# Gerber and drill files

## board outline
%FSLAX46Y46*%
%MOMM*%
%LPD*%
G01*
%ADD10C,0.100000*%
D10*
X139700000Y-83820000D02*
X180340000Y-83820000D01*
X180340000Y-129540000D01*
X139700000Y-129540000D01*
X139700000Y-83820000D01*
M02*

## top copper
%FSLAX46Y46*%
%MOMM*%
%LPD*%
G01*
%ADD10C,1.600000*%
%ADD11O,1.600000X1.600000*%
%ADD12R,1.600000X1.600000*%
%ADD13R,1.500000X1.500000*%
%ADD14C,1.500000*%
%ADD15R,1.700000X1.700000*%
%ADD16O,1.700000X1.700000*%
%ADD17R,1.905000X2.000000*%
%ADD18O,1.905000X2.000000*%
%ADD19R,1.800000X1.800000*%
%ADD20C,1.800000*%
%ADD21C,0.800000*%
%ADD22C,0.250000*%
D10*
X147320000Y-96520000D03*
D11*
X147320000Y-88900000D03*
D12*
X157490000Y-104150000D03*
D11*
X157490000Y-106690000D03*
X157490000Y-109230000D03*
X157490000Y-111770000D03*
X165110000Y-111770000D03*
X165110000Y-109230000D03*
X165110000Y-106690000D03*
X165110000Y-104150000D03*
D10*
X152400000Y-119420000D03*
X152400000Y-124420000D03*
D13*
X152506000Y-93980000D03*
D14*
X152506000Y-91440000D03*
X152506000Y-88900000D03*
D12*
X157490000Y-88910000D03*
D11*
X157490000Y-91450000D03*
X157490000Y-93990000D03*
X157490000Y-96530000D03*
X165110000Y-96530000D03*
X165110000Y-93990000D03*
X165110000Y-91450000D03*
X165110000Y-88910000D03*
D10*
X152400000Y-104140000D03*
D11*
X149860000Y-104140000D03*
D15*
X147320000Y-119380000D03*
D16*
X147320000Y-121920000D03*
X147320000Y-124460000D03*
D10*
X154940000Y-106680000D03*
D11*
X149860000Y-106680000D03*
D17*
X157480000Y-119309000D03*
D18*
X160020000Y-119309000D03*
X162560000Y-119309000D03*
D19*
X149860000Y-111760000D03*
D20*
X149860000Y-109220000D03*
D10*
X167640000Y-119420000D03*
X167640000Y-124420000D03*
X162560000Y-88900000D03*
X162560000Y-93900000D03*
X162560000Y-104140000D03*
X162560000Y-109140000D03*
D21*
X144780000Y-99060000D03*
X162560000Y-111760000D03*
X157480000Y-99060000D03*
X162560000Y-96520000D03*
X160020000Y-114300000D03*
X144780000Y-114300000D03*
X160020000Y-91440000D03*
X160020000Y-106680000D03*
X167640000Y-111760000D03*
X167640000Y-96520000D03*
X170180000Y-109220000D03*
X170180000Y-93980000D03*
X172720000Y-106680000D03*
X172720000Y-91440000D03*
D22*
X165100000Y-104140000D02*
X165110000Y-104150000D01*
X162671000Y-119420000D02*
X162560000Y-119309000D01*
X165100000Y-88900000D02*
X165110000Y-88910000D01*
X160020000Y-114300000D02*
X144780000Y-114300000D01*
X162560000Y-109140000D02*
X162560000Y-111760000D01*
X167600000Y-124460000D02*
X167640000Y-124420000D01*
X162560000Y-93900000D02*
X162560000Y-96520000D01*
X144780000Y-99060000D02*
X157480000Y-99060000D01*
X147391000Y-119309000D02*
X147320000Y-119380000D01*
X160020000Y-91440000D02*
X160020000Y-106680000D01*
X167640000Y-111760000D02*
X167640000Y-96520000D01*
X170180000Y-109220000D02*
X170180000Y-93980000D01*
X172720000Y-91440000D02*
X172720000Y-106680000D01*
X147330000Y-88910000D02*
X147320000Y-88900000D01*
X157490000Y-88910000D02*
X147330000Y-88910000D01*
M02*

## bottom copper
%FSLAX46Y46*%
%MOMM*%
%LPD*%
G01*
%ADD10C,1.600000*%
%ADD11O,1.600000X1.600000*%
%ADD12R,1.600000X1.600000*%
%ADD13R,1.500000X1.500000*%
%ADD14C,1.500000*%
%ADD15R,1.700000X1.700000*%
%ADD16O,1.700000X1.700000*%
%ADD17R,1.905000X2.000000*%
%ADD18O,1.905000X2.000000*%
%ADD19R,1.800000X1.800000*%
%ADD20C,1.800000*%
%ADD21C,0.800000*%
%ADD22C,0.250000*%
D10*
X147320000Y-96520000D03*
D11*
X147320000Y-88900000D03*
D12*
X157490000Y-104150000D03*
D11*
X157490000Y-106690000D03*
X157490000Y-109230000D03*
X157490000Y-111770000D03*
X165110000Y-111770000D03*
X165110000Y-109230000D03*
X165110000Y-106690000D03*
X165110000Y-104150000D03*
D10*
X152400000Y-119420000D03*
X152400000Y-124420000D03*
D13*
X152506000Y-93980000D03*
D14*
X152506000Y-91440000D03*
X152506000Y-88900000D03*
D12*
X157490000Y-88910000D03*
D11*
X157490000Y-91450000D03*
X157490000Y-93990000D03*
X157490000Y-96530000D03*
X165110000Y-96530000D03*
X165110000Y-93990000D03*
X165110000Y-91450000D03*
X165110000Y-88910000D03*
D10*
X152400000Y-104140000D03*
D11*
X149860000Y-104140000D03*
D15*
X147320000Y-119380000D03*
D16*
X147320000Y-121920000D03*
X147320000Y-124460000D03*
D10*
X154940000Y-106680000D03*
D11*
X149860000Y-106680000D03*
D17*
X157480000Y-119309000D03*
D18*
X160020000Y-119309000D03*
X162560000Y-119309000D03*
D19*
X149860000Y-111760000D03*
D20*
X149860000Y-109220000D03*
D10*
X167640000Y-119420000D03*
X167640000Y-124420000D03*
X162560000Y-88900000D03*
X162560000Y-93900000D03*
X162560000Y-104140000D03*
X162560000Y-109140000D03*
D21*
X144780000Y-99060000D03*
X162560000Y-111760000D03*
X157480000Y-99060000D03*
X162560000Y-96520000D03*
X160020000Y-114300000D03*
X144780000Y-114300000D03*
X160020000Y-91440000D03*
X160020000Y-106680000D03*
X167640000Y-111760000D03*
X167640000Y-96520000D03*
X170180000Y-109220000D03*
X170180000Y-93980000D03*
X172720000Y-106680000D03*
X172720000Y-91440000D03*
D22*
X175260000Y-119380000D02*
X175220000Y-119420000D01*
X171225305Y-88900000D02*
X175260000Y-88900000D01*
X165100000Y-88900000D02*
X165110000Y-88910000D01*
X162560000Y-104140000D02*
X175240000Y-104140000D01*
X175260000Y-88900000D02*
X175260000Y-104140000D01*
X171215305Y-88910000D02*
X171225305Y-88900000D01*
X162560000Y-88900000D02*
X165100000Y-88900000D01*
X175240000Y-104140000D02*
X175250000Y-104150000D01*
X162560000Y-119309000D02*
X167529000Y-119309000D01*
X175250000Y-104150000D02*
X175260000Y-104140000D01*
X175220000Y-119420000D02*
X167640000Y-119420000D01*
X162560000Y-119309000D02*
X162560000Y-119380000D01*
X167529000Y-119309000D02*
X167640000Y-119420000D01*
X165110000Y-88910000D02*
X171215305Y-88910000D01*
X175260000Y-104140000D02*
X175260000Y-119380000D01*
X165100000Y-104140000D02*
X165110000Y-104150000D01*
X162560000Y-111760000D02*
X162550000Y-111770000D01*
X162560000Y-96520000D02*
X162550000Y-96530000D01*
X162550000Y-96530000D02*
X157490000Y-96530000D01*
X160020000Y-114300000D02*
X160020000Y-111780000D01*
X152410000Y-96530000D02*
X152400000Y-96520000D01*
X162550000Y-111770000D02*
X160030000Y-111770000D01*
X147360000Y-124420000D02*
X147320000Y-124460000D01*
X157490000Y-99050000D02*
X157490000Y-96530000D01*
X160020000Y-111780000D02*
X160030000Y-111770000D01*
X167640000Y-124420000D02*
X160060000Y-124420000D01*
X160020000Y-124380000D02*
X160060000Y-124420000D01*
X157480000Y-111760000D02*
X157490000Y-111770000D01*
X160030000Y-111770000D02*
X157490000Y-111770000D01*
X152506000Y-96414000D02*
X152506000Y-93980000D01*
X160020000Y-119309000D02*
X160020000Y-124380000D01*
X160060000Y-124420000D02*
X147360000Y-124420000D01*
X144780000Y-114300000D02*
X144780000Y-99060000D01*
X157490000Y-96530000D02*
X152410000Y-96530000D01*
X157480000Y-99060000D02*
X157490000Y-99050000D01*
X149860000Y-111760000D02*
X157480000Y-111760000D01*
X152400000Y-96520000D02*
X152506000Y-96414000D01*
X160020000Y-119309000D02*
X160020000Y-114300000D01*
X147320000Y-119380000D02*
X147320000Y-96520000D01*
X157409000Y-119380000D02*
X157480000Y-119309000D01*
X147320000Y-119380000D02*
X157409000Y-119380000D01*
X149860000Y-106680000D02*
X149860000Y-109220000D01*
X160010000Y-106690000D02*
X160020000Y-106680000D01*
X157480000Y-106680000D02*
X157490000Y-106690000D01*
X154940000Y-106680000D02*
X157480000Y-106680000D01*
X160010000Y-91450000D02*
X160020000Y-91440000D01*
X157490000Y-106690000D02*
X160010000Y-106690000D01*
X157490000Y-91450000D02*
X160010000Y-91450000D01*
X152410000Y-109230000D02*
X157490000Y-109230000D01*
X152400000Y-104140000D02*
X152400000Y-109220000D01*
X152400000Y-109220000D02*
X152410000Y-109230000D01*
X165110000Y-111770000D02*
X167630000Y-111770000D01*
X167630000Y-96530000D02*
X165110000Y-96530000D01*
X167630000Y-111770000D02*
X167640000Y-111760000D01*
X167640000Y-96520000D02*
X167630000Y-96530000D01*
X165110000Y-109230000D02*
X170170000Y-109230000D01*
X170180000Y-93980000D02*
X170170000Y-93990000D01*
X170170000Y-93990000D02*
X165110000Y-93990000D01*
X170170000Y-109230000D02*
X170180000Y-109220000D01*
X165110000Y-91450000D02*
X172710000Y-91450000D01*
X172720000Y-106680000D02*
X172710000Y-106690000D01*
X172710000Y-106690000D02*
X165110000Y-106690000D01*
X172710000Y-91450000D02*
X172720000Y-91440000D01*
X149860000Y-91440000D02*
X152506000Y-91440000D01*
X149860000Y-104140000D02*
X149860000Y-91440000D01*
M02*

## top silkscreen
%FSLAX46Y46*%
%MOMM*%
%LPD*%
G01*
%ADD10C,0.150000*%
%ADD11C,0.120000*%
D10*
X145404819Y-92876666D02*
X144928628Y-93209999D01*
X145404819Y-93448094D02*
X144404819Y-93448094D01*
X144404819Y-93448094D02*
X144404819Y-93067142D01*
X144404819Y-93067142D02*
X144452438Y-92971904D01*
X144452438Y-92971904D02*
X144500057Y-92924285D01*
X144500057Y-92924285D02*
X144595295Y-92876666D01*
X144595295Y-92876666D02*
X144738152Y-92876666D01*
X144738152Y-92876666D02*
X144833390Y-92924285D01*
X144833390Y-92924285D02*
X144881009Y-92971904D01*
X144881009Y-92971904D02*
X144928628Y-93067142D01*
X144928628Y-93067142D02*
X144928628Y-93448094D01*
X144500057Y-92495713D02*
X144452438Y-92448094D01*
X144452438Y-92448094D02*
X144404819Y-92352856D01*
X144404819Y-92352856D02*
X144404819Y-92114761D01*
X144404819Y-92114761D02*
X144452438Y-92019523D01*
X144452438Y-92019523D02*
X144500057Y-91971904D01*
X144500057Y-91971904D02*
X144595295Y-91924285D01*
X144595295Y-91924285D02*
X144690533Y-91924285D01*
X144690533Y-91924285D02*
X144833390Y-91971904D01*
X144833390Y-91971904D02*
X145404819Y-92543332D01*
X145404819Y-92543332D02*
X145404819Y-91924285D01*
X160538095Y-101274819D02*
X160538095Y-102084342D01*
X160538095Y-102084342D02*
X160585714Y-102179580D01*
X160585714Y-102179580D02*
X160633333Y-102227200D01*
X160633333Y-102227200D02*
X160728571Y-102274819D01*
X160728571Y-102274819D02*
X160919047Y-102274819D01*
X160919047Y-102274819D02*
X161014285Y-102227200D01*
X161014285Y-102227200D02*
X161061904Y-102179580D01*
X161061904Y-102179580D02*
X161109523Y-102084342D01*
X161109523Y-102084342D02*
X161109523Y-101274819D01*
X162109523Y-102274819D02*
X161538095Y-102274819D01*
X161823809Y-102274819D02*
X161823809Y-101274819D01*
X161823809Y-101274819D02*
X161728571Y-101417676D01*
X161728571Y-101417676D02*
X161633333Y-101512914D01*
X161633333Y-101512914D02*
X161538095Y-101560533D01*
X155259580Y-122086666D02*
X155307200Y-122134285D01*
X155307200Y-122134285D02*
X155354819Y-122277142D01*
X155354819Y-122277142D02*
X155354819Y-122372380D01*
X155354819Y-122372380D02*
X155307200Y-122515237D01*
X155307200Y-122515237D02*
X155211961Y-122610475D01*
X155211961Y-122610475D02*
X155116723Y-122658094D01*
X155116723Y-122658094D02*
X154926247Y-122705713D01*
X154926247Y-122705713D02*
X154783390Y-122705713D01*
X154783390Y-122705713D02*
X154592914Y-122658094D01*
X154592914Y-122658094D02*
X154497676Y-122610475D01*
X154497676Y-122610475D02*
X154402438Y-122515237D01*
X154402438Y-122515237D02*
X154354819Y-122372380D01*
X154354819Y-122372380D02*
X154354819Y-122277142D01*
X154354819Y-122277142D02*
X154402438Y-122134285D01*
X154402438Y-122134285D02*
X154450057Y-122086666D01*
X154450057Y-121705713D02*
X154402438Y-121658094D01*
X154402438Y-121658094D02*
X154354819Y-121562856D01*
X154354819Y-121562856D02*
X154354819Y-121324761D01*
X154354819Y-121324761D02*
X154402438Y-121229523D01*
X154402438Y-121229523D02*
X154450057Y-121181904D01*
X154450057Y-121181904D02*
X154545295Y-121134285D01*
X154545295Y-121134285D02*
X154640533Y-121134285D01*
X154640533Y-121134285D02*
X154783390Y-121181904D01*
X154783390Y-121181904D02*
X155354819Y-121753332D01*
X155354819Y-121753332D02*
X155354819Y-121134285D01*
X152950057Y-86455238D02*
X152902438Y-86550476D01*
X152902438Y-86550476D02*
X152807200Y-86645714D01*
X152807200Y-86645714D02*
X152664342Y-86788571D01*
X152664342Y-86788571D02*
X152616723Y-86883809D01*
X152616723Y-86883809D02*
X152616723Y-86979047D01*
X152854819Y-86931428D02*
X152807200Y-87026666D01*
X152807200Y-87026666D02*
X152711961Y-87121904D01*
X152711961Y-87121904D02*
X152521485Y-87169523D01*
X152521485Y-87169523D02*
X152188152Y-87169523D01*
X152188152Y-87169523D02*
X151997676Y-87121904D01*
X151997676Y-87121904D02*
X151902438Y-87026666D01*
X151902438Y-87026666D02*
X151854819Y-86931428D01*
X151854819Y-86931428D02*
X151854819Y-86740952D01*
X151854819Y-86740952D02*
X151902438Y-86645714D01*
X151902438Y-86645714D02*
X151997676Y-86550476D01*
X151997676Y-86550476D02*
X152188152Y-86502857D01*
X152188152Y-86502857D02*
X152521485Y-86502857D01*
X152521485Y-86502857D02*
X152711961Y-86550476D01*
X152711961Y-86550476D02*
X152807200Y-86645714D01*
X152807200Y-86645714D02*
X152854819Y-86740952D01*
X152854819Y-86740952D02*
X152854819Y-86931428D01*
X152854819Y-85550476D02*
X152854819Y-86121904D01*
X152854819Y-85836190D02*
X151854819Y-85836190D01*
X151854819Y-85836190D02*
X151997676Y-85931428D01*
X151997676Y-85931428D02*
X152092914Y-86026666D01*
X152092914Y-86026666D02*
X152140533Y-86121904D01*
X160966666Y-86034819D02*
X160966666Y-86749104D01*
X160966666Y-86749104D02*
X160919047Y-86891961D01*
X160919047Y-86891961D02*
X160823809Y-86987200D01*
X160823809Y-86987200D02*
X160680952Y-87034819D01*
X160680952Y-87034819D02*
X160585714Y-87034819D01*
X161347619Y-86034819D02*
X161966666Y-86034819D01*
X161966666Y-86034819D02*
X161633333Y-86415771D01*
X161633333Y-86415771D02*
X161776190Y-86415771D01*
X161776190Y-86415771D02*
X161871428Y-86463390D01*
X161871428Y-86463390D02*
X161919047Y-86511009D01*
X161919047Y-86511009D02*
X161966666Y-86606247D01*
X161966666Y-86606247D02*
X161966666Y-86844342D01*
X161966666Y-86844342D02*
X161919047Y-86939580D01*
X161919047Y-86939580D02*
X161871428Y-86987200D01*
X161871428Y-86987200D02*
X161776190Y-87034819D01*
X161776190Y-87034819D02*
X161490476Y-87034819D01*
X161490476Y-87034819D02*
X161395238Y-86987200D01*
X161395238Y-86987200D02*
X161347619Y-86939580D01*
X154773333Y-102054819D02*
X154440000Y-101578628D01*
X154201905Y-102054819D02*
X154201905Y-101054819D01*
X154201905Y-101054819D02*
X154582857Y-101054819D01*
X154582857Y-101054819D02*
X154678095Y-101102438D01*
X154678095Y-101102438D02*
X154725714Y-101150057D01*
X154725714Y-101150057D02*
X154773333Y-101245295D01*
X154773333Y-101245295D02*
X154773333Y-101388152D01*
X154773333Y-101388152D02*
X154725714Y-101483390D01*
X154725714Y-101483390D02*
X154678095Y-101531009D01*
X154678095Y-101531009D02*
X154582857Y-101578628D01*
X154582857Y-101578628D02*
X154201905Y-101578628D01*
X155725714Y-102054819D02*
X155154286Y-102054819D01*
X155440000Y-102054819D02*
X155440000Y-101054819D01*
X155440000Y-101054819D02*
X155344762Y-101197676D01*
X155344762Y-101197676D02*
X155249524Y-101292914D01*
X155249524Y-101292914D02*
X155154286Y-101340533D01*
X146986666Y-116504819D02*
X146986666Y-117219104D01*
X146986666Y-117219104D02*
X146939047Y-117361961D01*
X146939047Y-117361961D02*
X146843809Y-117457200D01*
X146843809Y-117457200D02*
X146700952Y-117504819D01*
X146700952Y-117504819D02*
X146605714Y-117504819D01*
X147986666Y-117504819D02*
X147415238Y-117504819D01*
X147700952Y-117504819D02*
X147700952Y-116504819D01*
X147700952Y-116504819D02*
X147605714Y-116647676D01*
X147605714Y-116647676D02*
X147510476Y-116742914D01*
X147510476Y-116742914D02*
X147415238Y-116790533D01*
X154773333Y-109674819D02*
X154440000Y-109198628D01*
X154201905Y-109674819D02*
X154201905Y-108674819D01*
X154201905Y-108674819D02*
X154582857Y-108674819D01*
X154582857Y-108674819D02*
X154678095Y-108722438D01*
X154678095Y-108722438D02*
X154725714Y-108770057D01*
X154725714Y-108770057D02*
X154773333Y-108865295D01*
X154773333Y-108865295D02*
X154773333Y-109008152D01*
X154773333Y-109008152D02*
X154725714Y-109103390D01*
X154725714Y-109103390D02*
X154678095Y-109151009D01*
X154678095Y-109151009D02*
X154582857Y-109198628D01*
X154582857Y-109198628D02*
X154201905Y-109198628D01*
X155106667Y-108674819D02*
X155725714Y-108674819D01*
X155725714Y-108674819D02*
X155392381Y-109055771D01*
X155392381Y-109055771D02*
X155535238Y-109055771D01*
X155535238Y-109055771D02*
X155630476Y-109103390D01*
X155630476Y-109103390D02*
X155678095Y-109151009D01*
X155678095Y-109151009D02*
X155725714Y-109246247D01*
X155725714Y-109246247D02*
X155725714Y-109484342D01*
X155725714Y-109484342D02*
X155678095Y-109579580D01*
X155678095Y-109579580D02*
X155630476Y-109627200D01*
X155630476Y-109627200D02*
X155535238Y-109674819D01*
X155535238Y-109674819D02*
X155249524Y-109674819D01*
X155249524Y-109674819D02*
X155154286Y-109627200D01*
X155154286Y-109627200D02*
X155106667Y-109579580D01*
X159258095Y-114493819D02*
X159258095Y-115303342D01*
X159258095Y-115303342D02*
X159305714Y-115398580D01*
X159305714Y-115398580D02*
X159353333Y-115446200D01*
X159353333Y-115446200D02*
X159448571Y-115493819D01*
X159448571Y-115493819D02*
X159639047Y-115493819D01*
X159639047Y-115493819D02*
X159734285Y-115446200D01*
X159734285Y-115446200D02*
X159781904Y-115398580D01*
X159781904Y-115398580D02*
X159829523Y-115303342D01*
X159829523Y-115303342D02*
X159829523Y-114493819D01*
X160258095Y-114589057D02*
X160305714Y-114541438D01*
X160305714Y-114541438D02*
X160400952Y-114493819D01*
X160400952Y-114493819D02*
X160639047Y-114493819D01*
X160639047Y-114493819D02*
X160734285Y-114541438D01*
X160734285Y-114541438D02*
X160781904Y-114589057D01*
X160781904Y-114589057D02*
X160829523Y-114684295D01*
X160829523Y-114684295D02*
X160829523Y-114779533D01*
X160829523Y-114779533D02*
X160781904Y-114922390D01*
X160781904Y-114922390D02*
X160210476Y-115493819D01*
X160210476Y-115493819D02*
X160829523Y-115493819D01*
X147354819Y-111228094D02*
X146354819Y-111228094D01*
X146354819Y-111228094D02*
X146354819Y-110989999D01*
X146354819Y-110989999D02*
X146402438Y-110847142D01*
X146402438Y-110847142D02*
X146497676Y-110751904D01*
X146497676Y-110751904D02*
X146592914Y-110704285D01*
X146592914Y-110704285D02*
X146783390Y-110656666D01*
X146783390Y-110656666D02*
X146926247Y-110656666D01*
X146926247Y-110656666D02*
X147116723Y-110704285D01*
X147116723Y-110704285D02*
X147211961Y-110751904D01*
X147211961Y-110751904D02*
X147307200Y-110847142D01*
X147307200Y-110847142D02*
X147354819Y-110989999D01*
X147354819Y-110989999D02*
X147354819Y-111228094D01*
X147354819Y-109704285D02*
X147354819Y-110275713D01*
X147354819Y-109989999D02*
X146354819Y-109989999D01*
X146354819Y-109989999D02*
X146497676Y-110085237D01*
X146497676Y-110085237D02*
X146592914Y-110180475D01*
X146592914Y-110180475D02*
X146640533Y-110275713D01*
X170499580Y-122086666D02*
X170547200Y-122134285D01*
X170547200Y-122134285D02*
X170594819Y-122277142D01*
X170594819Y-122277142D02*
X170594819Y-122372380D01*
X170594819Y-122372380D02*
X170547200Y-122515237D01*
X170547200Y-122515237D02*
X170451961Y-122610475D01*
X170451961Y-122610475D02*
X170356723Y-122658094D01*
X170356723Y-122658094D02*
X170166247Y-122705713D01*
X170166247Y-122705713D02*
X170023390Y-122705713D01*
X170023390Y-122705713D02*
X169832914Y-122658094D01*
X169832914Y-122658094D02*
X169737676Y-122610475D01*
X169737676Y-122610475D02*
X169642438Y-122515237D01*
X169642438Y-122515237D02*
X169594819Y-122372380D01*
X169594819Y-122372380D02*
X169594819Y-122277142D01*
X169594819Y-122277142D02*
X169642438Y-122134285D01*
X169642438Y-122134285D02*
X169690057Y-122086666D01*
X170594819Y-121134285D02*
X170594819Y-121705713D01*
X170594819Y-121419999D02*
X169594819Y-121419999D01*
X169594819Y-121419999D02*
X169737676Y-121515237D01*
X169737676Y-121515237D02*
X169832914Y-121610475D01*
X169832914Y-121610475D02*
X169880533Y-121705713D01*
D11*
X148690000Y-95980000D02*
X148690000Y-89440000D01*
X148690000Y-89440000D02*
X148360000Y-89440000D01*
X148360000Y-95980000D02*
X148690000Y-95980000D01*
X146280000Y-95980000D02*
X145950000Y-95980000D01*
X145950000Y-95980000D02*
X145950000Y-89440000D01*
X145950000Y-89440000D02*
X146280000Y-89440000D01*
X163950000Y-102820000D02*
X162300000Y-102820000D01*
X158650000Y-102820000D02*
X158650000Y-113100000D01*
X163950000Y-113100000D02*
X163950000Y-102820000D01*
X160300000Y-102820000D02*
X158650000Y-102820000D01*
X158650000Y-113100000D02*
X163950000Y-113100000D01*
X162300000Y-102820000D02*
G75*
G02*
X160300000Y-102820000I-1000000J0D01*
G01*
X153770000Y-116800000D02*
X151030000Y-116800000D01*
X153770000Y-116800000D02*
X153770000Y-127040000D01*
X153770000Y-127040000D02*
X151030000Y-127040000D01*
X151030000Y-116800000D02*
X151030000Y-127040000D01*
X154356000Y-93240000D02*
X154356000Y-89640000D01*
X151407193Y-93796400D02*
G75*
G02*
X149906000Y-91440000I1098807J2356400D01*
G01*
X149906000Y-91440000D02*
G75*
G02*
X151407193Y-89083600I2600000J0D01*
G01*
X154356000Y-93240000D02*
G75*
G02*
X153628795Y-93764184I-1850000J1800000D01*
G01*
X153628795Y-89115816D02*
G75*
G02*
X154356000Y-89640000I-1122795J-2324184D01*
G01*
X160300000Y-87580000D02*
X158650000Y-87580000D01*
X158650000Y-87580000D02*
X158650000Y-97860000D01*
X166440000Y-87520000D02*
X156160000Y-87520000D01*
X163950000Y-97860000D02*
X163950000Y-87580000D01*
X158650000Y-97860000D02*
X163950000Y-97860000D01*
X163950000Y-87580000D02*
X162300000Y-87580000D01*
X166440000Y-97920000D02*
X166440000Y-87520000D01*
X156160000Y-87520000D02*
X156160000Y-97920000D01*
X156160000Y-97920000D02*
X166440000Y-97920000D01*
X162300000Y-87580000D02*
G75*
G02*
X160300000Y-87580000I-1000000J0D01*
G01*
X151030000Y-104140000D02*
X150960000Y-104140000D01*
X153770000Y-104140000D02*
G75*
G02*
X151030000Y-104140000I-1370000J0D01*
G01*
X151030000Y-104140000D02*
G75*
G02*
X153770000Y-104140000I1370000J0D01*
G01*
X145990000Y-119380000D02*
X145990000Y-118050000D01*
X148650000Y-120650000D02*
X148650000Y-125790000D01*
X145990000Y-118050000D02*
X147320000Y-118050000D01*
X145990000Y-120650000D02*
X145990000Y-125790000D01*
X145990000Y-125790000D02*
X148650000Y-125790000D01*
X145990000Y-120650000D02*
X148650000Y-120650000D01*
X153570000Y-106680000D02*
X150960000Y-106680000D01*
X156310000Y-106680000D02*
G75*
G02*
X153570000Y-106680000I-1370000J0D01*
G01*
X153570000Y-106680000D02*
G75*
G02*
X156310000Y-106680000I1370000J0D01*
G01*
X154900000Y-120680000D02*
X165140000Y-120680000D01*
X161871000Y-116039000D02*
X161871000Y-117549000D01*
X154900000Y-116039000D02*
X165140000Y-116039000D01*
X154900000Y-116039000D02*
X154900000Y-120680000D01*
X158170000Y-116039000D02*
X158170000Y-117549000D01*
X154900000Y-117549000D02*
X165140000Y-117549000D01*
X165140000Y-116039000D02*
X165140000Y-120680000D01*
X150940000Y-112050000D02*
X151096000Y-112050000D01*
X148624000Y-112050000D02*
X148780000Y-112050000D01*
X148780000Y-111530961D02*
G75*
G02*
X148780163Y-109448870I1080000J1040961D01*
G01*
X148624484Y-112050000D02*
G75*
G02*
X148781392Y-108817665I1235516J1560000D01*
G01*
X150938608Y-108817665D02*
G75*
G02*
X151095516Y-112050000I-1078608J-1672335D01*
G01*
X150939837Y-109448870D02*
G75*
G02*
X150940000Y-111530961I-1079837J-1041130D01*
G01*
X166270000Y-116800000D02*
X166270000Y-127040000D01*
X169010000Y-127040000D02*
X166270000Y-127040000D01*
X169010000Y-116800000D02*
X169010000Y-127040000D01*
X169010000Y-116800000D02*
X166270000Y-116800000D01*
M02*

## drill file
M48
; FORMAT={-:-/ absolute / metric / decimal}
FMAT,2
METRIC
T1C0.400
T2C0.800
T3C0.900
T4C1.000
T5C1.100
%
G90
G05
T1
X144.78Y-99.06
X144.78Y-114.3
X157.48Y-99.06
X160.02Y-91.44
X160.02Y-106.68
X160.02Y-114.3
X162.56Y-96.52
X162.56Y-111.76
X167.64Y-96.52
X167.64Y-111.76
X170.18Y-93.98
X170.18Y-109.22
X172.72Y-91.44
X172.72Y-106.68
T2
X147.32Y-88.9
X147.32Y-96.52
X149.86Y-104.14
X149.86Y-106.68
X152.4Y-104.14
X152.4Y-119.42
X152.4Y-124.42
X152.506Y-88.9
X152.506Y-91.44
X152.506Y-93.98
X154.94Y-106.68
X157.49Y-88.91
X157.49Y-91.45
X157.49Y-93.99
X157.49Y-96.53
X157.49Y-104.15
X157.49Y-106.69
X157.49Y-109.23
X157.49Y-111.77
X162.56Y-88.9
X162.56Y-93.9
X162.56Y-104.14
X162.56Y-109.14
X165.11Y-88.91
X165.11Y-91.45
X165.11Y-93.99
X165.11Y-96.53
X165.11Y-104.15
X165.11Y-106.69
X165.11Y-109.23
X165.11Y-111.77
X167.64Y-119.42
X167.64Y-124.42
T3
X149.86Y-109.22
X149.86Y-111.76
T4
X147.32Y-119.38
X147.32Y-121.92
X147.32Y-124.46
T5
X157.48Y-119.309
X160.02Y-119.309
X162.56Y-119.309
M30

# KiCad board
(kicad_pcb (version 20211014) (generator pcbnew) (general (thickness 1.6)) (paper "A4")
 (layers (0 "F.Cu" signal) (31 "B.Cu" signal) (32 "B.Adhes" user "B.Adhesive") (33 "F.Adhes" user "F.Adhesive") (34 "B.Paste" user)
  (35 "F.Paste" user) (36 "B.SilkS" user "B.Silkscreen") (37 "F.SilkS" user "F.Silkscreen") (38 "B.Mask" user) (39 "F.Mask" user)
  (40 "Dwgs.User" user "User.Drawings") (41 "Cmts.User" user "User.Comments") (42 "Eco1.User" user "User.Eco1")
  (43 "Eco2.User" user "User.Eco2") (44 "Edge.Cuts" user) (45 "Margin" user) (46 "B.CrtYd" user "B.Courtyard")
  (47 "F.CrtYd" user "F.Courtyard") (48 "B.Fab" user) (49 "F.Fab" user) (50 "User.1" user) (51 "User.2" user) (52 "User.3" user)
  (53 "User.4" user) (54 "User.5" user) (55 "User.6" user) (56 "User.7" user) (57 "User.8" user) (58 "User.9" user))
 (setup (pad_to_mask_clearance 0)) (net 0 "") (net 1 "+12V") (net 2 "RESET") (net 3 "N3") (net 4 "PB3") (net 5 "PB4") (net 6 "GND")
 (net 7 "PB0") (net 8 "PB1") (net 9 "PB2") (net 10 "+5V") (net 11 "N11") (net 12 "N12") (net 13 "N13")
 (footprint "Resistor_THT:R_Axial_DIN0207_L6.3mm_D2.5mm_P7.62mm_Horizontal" (layer "F.Cu") (at 147.32 96.52 90)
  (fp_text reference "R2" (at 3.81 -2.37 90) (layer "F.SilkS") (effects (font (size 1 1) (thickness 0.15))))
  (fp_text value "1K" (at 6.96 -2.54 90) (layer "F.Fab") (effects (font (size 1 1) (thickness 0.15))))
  (fp_line (start 0.54 1.37) (end 7.08 1.37) (layer "F.SilkS") (width 0.12))
  (fp_line (start 7.08 1.37) (end 7.08 1.04) (layer "F.SilkS") (width 0.12))
  (fp_line (start 0.54 1.04) (end 0.54 1.37) (layer "F.SilkS") (width 0.12))
  (fp_line (start 0.54 -1.04) (end 0.54 -1.37) (layer "F.SilkS") (width 0.12))
  (fp_line (start 0.54 -1.37) (end 7.08 -1.37) (layer "F.SilkS") (width 0.12))
  (fp_line (start 7.08 -1.37) (end 7.08 -1.04) (layer "F.SilkS") (width 0.12))
  (pad "1" thru_hole circle (at 0 0 90) (size 1.6 1.6) (drill 0.8) (layers *.Cu *.Mask) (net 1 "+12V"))
  (pad "2" thru_hole oval (at 7.62 0 90) (size 1.6 1.6) (drill 0.8) (layers *.Cu *.Mask) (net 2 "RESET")))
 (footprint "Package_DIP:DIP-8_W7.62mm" (layer "F.Cu") (at 157.49 104.15)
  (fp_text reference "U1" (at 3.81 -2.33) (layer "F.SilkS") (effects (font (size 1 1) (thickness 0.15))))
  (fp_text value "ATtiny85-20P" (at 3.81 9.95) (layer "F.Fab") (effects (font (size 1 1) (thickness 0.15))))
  (fp_line (start 6.46 -1.33) (end 4.81 -1.33) (layer "F.SilkS") (width 0.12))
  (fp_line (start 1.16 -1.33) (end 1.16 8.95) (layer "F.SilkS") (width 0.12))
  (fp_line (start 6.46 8.95) (end 6.46 -1.33) (layer "F.SilkS") (width 0.12))
  (fp_line (start 2.81 -1.33) (end 1.16 -1.33) (layer "F.SilkS") (width 0.12))
  (fp_line (start 1.16 8.95) (end 6.46 8.95) (layer "F.SilkS") (width 0.12))
  (fp_arc (start 4.81 -1.33) (mid 3.81 -0.33) (end 2.81 -1.33) (layer "F.SilkS") (width 0.12))
  (pad "1" thru_hole rect (at 0 0) (size 1.6 1.6) (drill 0.8) (layers *.Cu *.Mask) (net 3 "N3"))
  (pad "2" thru_hole oval (at 0 2.54) (size 1.6 1.6) (drill 0.8) (layers *.Cu *.Mask) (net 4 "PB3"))
  (pad "3" thru_hole oval (at 0 5.08) (size 1.6 1.6) (drill 0.8) (layers *.Cu *.Mask) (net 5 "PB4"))
  (pad "4" thru_hole oval (at 0 7.62) (size 1.6 1.6) (drill 0.8) (layers *.Cu *.Mask) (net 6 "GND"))
  (pad "5" thru_hole oval (at 7.62 7.62) (size 1.6 1.6) (drill 0.8) (layers *.Cu *.Mask) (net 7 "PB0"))
  (pad "6" thru_hole oval (at 7.62 5.08) (size 1.6 1.6) (drill 0.8) (layers *.Cu *.Mask) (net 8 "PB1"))
  (pad "7" thru_hole oval (at 7.62 2.54) (size 1.6 1.6) (drill 0.8) (layers *.Cu *.Mask) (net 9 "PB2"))
  (pad "8" thru_hole oval (at 7.62 0) (size 1.6 1.6) (drill 0.8) (layers *.Cu *.Mask) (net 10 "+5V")))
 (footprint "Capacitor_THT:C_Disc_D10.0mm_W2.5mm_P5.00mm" (layer "F.Cu") (at 152.4 119.42 -90)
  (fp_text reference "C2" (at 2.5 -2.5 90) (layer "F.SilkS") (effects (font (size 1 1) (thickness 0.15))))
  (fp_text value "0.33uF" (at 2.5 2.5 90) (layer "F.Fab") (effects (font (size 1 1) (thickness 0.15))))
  (fp_line (start -2.62 -1.37) (end -2.62 1.37) (layer "F.SilkS") (width 0.12))
  (fp_line (start -2.62 -1.37) (end 7.62 -1.37) (layer "F.SilkS") (width 0.12))
  (fp_line (start 7.62 -1.37) (end 7.62 1.37) (layer "F.SilkS") (width 0.12))
  (fp_line (start -2.62 1.37) (end 7.62 1.37) (layer "F.SilkS") (width 0.12))
  (pad "1" thru_hole circle (at 0 0 270) (size 1.6 1.6) (drill 0.8) (layers *.Cu *.Mask) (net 1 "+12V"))
  (pad "2" thru_hole circle (at 5 0 270) (size 1.6 1.6) (drill 0.8) (layers *.Cu *.Mask) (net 6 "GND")))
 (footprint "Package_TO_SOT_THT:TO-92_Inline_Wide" (layer "F.Cu") (at 152.506 93.98 90)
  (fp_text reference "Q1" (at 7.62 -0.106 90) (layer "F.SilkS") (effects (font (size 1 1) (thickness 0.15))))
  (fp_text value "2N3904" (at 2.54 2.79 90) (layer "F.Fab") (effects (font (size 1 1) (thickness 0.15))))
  (fp_line (start 0.74 1.85) (end 4.34 1.85) (layer "F.SilkS") (width 0.12))
  (fp_arc (start 0.1836 -1.098807) (mid 1.143021 -2.192817) (end 2.54 -2.6) (layer "F.SilkS") (width 0.12))
  (fp_arc (start 2.54 -2.6) (mid 3.936979 -2.192818) (end 4.8964 -1.098807) (layer "F.SilkS") (width 0.12))
  (fp_arc (start 0.74 1.85) (mid 0.446097 1.509328) (end 0.215816 1.122795) (layer "F.SilkS") (width 0.12))
  (fp_arc (start 4.864184 1.122795) (mid 4.633903 1.509328) (end 4.34 1.85) (layer "F.SilkS") (width 0.12))
  (pad "1" thru_hole rect (at 0 0 90) (size 1.5 1.5) (drill 0.8) (layers *.Cu *.Mask) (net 6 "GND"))
  (pad "2" thru_hole circle (at 2.54 0 90) (size 1.5 1.5) (drill 0.8) (layers *.Cu *.Mask) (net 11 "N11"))
  (pad "3" thru_hole circle (at 5.08 0 90) (size 1.5 1.5) (drill 0.8) (layers *.Cu *.Mask) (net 2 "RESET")))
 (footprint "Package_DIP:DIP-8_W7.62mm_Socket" (layer "F.Cu") (at 157.49 88.91)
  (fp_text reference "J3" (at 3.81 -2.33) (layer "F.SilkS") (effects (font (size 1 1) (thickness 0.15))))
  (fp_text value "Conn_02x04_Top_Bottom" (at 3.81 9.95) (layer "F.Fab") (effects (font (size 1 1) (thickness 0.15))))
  (fp_line (start 2.81 -1.33) (end 1.16 -1.33) (layer "F.SilkS") (width 0.12))
  (fp_line (start 1.16 -1.33) (end 1.16 8.95) (layer "F.SilkS") (width 0.12))
  (fp_line (start 8.95 -1.39) (end -1.33 -1.39) (layer "F.SilkS") (width 0.12))
  (fp_line (start 6.46 8.95) (end 6.46 -1.33) (layer "F.SilkS") (width 0.12))
  (fp_line (start 1.16 8.95) (end 6.46 8.95) (layer "F.SilkS") (width 0.12))
  (fp_line (start 6.46 -1.33) (end 4.81 -1.33) (layer "F.SilkS") (width 0.12))
  (fp_line (start 8.95 9.01) (end 8.95 -1.39) (layer "F.SilkS") (width 0.12))
  (fp_line (start -1.33 -1.39) (end -1.33 9.01) (layer "F.SilkS") (width 0.12))
  (fp_line (start -1.33 9.01) (end 8.95 9.01) (layer "F.SilkS") (width 0.12))
  (fp_arc (start 4.81 -1.33) (mid 3.81 -0.33) (end 2.81 -1.33) (layer "F.SilkS") (width 0.12))
  (pad "1" thru_hole rect (at 0 0) (size 1.6 1.6) (drill 0.8) (layers *.Cu *.Mask) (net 2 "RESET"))
  (pad "2" thru_hole oval (at 0 2.54) (size 1.6 1.6) (drill 0.8) (layers *.Cu *.Mask) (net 4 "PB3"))
  (pad "3" thru_hole oval (at 0 5.08) (size 1.6 1.6) (drill 0.8) (layers *.Cu *.Mask) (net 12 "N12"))
  (pad "4" thru_hole oval (at 0 7.62) (size 1.6 1.6) (drill 0.8) (layers *.Cu *.Mask) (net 6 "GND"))
  (pad "5" thru_hole oval (at 7.62 7.62) (size 1.6 1.6) (drill 0.8) (layers *.Cu *.Mask) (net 7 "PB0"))
  (pad "6" thru_hole oval (at 7.62 5.08) (size 1.6 1.6) (drill 0.8) (layers *.Cu *.Mask) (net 8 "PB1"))
  (pad "7" thru_hole oval (at 7.62 2.54) (size 1.6 1.6) (drill 0.8) (layers *.Cu *.Mask) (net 9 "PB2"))
  (pad "8" thru_hole oval (at 7.62 0) (size 1.6 1.6) (drill 0.8) (layers *.Cu *.Mask) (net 10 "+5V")))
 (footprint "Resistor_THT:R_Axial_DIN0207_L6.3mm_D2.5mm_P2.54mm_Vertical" (layer "F.Cu") (at 152.4 104.14 180)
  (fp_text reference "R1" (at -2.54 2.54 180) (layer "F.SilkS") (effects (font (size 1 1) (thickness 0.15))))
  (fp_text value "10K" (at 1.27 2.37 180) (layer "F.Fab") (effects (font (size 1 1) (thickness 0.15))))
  (fp_line (start 1.37 0) (end 1.44 0) (layer "F.SilkS") (width 0.12))
  (fp_circle (center 0 0) (end 1.37 0) (layer "F.SilkS") (width 0.12) (fill none))
  (pad "1" thru_hole circle (at 0 0 180) (size 1.6 1.6) (drill 0.8) (layers *.Cu *.Mask) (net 5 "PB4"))
  (pad "2" thru_hole oval (at 2.54 0 180) (size 1.6 1.6) (drill 0.8) (layers *.Cu *.Mask) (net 11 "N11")))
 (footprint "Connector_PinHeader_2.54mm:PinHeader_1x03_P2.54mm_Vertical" (layer "F.Cu") (at 147.32 119.38)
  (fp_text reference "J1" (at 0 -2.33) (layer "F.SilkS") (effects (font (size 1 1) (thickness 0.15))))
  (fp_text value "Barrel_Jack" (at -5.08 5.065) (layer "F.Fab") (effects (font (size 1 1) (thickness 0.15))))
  (fp_line (start -1.33 0) (end -1.33 -1.33) (layer "F.SilkS") (width 0.12))
  (fp_line (start 1.33 1.27) (end 1.33 6.41) (layer "F.SilkS") (width 0.12))
  (fp_line (start -1.33 -1.33) (end 0 -1.33) (layer "F.SilkS") (width 0.12))
  (fp_line (start -1.33 1.27) (end -1.33 6.41) (layer "F.SilkS") (width 0.12))
  (fp_line (start -1.33 6.41) (end 1.33 6.41) (layer "F.SilkS") (width 0.12))
  (fp_line (start -1.33 1.27) (end 1.33 1.27) (layer "F.SilkS") (width 0.12))
  (pad "1" thru_hole rect (at 0 0) (size 1.7 1.7) (drill 1) (layers *.Cu *.Mask) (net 1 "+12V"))
  (pad "2" thru_hole oval (at 0 2.54) (size 1.7 1.7) (drill 1) (layers *.Cu *.Mask))
  (pad "3" thru_hole oval (at 0 5.08) (size 1.7 1.7) (drill 1) (layers *.Cu *.Mask) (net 6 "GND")))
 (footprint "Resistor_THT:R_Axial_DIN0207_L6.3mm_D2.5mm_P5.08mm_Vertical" (layer "F.Cu") (at 154.94 106.68 180)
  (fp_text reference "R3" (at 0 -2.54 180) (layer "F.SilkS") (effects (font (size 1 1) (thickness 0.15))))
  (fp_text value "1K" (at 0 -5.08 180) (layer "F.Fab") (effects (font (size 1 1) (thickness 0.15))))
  (fp_line (start 1.37 0) (end 3.98 0) (layer "F.SilkS") (width 0.12))
  (fp_circle (center 0 0) (end 1.37 0) (layer "F.SilkS") (width 0.12) (fill none))
  (pad "1" thru_hole circle (at 0 0 180) (size 1.6 1.6) (drill 0.8) (layers *.Cu *.Mask) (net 4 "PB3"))
  (pad "2" thru_hole oval (at 5.08 0 180) (size 1.6 1.6) (drill 0.8) (layers *.Cu *.Mask) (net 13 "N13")))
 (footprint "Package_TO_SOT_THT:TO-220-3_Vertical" (layer "F.Cu") (at 157.48 119.309)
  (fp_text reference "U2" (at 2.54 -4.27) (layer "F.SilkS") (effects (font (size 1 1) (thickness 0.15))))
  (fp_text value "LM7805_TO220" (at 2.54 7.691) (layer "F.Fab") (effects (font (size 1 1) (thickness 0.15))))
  (fp_line (start -2.58 1.371) (end 7.66 1.371) (layer "F.SilkS") (width 0.12))
  (fp_line (start 4.391 -3.27) (end 4.391 -1.76) (layer "F.SilkS") (width 0.12))
  (fp_line (start -2.58 -3.27) (end 7.66 -3.27) (layer "F.SilkS") (width 0.12))
  (fp_line (start -2.58 -3.27) (end -2.58 1.371) (layer "F.SilkS") (width 0.12))
  (fp_line (start 0.69 -3.27) (end 0.69 -1.76) (layer "F.SilkS") (width 0.12))
  (fp_line (start -2.58 -1.76) (end 7.66 -1.76) (layer "F.SilkS") (width 0.12))
  (fp_line (start 7.66 -3.27) (end 7.66 1.371) (layer "F.SilkS") (width 0.12))
  (pad "1" thru_hole rect (at 0 0) (size 1.905 2) (drill 1.1) (layers *.Cu *.Mask) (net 1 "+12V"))
  (pad "2" thru_hole oval (at 2.54 0) (size 1.905 2) (drill 1.1) (layers *.Cu *.Mask) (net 6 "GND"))
  (pad "3" thru_hole oval (at 5.08 0) (size 1.905 2) (drill 1.1) (layers *.Cu *.Mask) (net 10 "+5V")))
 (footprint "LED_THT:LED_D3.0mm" (layer "F.Cu") (at 149.86 111.76 90)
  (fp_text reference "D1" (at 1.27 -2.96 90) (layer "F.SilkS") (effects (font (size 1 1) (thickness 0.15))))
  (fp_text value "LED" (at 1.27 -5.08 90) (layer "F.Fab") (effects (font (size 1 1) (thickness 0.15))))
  (fp_line (start -0.29 1.08) (end -0.29 1.236) (layer "F.SilkS") (width 0.12))
  (fp_line (start -0.29 -1.236) (end -0.29 -1.08) (layer "F.SilkS") (width 0.12))
  (fp_arc (start 0.229039 -1.08) (mid 1.270117 -1.5) (end 2.31113 -1.079837) (layer "F.SilkS") (width 0.12))
  (fp_arc (start -0.29 -1.235516) (mid 1.366487 -1.987659) (end 2.942335 -1.078608) (layer "F.SilkS") (width 0.12))
  (fp_arc (start 2.942335 1.078608) (mid 1.366487 1.987659) (end -0.29 1.235516) (layer "F.SilkS") (width 0.12))
  (fp_arc (start 2.31113 1.079837) (mid 1.270117 1.5) (end 0.229039 1.08) (layer "F.SilkS") (width 0.12))
  (pad "1" thru_hole rect (at 0 0 90) (size 1.8 1.8) (drill 0.9) (layers *.Cu *.Mask) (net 6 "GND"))
  (pad "2" thru_hole circle (at 2.54 0 90) (size 1.8 1.8) (drill 0.9) (layers *.Cu *.Mask) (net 13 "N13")))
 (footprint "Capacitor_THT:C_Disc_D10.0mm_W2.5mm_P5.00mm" (layer "F.Cu") (at 167.64 119.42 -90)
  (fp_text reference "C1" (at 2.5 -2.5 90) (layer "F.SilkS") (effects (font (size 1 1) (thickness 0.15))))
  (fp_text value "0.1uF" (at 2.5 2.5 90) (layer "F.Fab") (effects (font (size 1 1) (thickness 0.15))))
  (fp_line (start -2.62 1.37) (end 7.62 1.37) (layer "F.SilkS") (width 0.12))
  (fp_line (start 7.62 -1.37) (end 7.62 1.37) (layer "F.SilkS") (width 0.12))
  (fp_line (start -2.62 -1.37) (end 7.62 -1.37) (layer "F.SilkS") (width 0.12))
  (fp_line (start -2.62 -1.37) (end -2.62 1.37) (layer "F.SilkS") (width 0.12))
  (pad "1" thru_hole circle (at 0 0 270) (size 1.6 1.6) (drill 0.8) (layers *.Cu *.Mask) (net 10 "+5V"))
  (pad "2" thru_hole circle (at 5 0 270) (size 1.6 1.6) (drill 0.8) (layers *.Cu *.Mask) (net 6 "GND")))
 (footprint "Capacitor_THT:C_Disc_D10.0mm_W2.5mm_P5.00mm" (layer "B.Cu") (at 162.56 88.9 -90)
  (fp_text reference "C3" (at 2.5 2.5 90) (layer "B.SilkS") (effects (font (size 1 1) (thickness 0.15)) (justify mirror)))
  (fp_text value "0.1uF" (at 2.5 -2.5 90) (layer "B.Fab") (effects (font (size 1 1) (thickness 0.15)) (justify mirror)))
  (pad "1" thru_hole circle (at 0 0 270) (size 1.6 1.6) (drill 0.8) (layers *.Cu *.Mask) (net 10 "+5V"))
  (pad "2" thru_hole circle (at 5 0 270) (size 1.6 1.6) (drill 0.8) (layers *.Cu *.Mask) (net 6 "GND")))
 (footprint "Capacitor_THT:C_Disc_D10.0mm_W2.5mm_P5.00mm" (layer "B.Cu") (at 162.56 104.14 -90)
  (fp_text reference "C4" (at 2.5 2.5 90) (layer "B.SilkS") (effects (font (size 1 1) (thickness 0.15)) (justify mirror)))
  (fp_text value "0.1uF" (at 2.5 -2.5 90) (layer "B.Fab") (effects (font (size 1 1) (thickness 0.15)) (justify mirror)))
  (pad "1" thru_hole circle (at 0 0 270) (size 1.6 1.6) (drill 0.8) (layers *.Cu *.Mask) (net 10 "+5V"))
  (pad "2" thru_hole circle (at 5 0 270) (size 1.6 1.6) (drill 0.8) (layers *.Cu *.Mask) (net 6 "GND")))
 (gr_rect (start 139.7 83.82) (end 180.34 129.54) (layer "Edge.Cuts") (width 0.1) (fill none))
 (segment (start 165.1 104.14) (end 165.11 104.15) (width 0.25) (layer "F.Cu") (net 10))
 (segment (start 162.671 119.42) (end 162.56 119.309) (width 0.25) (layer "F.Cu") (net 10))
 (segment (start 165.1 88.9) (end 165.11 88.91) (width 0.25) (layer "F.Cu") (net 10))
 (segment (start 175.26 119.38) (end 175.22 119.42) (width 0.25) (layer "B.Cu") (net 10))
 (segment (start 171.225305 88.9) (end 175.26 88.9) (width 0.25) (layer "B.Cu") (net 10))
 (segment (start 165.1 88.9) (end 165.11 88.91) (width 0.25) (layer "B.Cu") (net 10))
 (segment (start 162.56 104.14) (end 175.24 104.14) (width 0.25) (layer "B.Cu") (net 10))
 (segment (start 175.26 88.9) (end 175.26 104.14) (width 0.25) (layer "B.Cu") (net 10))
 (segment (start 171.215305 88.91) (end 171.225305 88.9) (width 0.25) (layer "B.Cu") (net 10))
 (segment (start 162.56 88.9) (end 165.1 88.9) (width 0.25) (layer "B.Cu") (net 10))
 (segment (start 175.24 104.14) (end 175.25 104.15) (width 0.25) (layer "B.Cu") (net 10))
 (segment (start 162.56 119.309) (end 167.529 119.309) (width 0.25) (layer "B.Cu") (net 10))
 (segment (start 175.25 104.15) (end 175.26 104.14) (width 0.25) (layer "B.Cu") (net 10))
 (segment (start 175.22 119.42) (end 167.64 119.42) (width 0.25) (layer "B.Cu") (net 10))
 (segment (start 162.56 119.309) (end 162.56 119.38) (width 0.25) (layer "B.Cu") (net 10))
 (segment (start 167.529 119.309) (end 167.64 119.42) (width 0.25) (layer "B.Cu") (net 10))
 (segment (start 165.11 88.91) (end 171.215305 88.91) (width 0.25) (layer "B.Cu") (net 10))
 (segment (start 175.26 104.14) (end 175.26 119.38) (width 0.25) (layer "B.Cu") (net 10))
 (segment (start 165.1 104.14) (end 165.11 104.15) (width 0.25) (layer "B.Cu") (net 10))
 (segment (start 160.02 114.3) (end 144.78 114.3) (width 0.25) (layer "F.Cu") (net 6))
 (segment (start 162.56 109.14) (end 162.56 111.76) (width 0.25) (layer "F.Cu") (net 6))
 (segment (start 167.6 124.46) (end 167.64 124.42) (width 0.25) (layer "F.Cu") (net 6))
 (segment (start 162.56 93.9) (end 162.56 96.52) (width 0.25) (layer "F.Cu") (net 6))
 (segment (start 144.78 99.06) (end 157.48 99.06) (width 0.25) (layer "F.Cu") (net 6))
 (via (at 144.78 99.06) (size 0.8) (drill 0.4) (layers "F.Cu" "B.Cu") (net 6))
 (via (at 162.56 111.76) (size 0.8) (drill 0.4) (layers "F.Cu" "B.Cu") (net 6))
 (via (at 157.48 99.06) (size 0.8) (drill 0.4) (layers "F.Cu" "B.Cu") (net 6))
 (via (at 162.56 96.52) (size 0.8) (drill 0.4) (layers "F.Cu" "B.Cu") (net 6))
 (via (at 160.02 114.3) (size 0.8) (drill 0.4) (layers "F.Cu" "B.Cu") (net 6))
 (via (at 144.78 114.3) (size 0.8) (drill 0.4) (layers "F.Cu" "B.Cu") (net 6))
 (segment (start 162.56 111.76) (end 162.55 111.77) (width 0.25) (layer "B.Cu") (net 6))
 (segment (start 162.56 96.52) (end 162.55 96.53) (width 0.25) (layer "B.Cu") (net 6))
 (segment (start 162.55 96.53) (end 157.49 96.53) (width 0.25) (layer "B.Cu") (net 6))
 (segment (start 160.02 114.3) (end 160.02 111.78) (width 0.25) (layer "B.Cu") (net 6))
 (segment (start 152.41 96.53) (end 152.4 96.52) (width 0.25) (layer "B.Cu") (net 6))
 (segment (start 162.55 111.77) (end 160.03 111.77) (width 0.25) (layer "B.Cu") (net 6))
 (segment (start 147.36 124.42) (end 147.32 124.46) (width 0.25) (layer "B.Cu") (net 6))
 (segment (start 157.49 99.05) (end 157.49 96.53) (width 0.25) (layer "B.Cu") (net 6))
 (segment (start 160.02 111.78) (end 160.03 111.77) (width 0.25) (layer "B.Cu") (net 6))
 (segment (start 167.64 124.42) (end 160.06 124.42) (width 0.25) (layer "B.Cu") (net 6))
 (segment (start 160.02 124.38) (end 160.06 124.42) (width 0.25) (layer "B.Cu") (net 6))
 (segment (start 157.48 111.76) (end 157.49 111.77) (width 0.25) (layer "B.Cu") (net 6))
 (segment (start 160.03 111.77) (end 157.49 111.77) (width 0.25) (layer "B.Cu") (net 6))
 (segment (start 152.506 96.414) (end 152.506 93.98) (width 0.25) (layer "B.Cu") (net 6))
 (segment (start 160.02 119.309) (end 160.02 124.38) (width 0.25) (layer "B.Cu") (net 6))
 (segment (start 160.06 124.42) (end 147.36 124.42) (width 0.25) (layer "B.Cu") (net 6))
 (segment (start 144.78 114.3) (end 144.78 99.06) (width 0.25) (layer "B.Cu") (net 6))
 (segment (start 157.49 96.53) (end 152.41 96.53) (width 0.25) (layer "B.Cu") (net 6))
 (segment (start 157.48 99.06) (end 157.49 99.05) (width 0.25) (layer "B.Cu") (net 6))
 (segment (start 149.86 111.76) (end 157.48 111.76) (width 0.25) (layer "B.Cu") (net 6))
 (segment (start 152.4 96.52) (end 152.506 96.414) (width 0.25) (layer "B.Cu") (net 6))
 (segment (start 160.02 119.309) (end 160.02 114.3) (width 0.25) (layer "B.Cu") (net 6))
 (segment (start 147.391 119.309) (end 147.32 119.38) (width 0.25) (layer "F.Cu") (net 1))
 (segment (start 147.32 119.38) (end 147.32 96.52) (width 0.25) (layer "B.Cu") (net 1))
 (segment (start 157.409 119.38) (end 157.48 119.309) (width 0.25) (layer "B.Cu") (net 1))
 (segment (start 147.32 119.38) (end 157.409 119.38) (width 0.25) (layer "B.Cu") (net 1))
 (segment (start 149.86 106.68) (end 149.86 109.22) (width 0.25) (layer "B.Cu") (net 13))
 (segment (start 160.02 91.44) (end 160.02 106.68) (width 0.25) (layer "F.Cu") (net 4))
 (via (at 160.02 91.44) (size 0.8) (drill 0.4) (layers "F.Cu" "B.Cu") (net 4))
 (via (at 160.02 106.68) (size 0.8) (drill 0.4) (layers "F.Cu" "B.Cu") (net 4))
 (segment (start 160.01 106.69) (end 160.02 106.68) (width 0.25) (layer "B.Cu") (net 4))
 (segment (start 157.48 106.68) (end 157.49 106.69) (width 0.25) (layer "B.Cu") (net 4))
 (segment (start 154.94 106.68) (end 157.48 106.68) (width 0.25) (layer "B.Cu") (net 4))
 (segment (start 160.01 91.45) (end 160.02 91.44) (width 0.25) (layer "B.Cu") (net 4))
 (segment (start 157.49 106.69) (end 160.01 106.69) (width 0.25) (layer "B.Cu") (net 4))
 (segment (start 157.49 91.45) (end 160.01 91.45) (width 0.25) (layer "B.Cu") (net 4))
 (segment (start 152.41 109.23) (end 157.49 109.23) (width 0.25) (layer "B.Cu") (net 5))
 (segment (start 152.4 104.14) (end 152.4 109.22) (width 0.25) (layer "B.Cu") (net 5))
 (segment (start 152.4 109.22) (end 152.41 109.23) (width 0.25) (layer "B.Cu") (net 5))
 (segment (start 167.64 111.76) (end 167.64 96.52) (width 0.25) (layer "F.Cu") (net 7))
 (via (at 167.64 111.76) (size 0.8) (drill 0.4) (layers "F.Cu" "B.Cu") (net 7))
 (via (at 167.64 96.52) (size 0.8) (drill 0.4) (layers "F.Cu" "B.Cu") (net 7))
 (segment (start 165.11 111.77) (end 167.63 111.77) (width 0.25) (layer "B.Cu") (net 7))
 (segment (start 167.63 96.53) (end 165.11 96.53) (width 0.25) (layer "B.Cu") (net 7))
 (segment (start 167.63 111.77) (end 167.64 111.76) (width 0.25) (layer "B.Cu") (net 7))
 (segment (start 167.64 96.52) (end 167.63 96.53) (width 0.25) (layer "B.Cu") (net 7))
 (segment (start 170.18 109.22) (end 170.18 93.98) (width 0.25) (layer "F.Cu") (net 8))
 (via (at 170.18 109.22) (size 0.8) (drill 0.4) (layers "F.Cu" "B.Cu") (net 8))
 (via (at 170.18 93.98) (size 0.8) (drill 0.4) (layers "F.Cu" "B.Cu") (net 8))
 (segment (start 165.11 109.23) (end 170.17 109.23) (width 0.25) (layer "B.Cu") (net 8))
 (segment (start 170.18 93.98) (end 170.17 93.99) (width 0.25) (layer "B.Cu") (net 8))
 (segment (start 170.17 93.99) (end 165.11 93.99) (width 0.25) (layer "B.Cu") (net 8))
 (segment (start 170.17 109.23) (end 170.18 109.22) (width 0.25) (layer "B.Cu") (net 8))
 (segment (start 172.72 91.44) (end 172.72 106.68) (width 0.25) (layer "F.Cu") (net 9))
 (via (at 172.72 106.68) (size 0.8) (drill 0.4) (layers "F.Cu" "B.Cu") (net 9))
 (via (at 172.72 91.44) (size 0.8) (drill 0.4) (layers "F.Cu" "B.Cu") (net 9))
 (segment (start 165.11 91.45) (end 172.71 91.45) (width 0.25) (layer "B.Cu") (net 9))
 (segment (start 172.72 106.68) (end 172.71 106.69) (width 0.25) (layer "B.Cu") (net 9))
 (segment (start 172.71 106.69) (end 165.11 106.69) (width 0.25) (layer "B.Cu") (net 9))
 (segment (start 172.71 91.45) (end 172.72 91.44) (width 0.25) (layer "B.Cu") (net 9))
 (segment (start 147.33 88.91) (end 147.32 88.9) (width 0.25) (layer "F.Cu") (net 2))
 (segment (start 157.49 88.91) (end 147.33 88.91) (width 0.25) (layer "F.Cu") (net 2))
 (segment (start 149.86 91.44) (end 152.506 91.44) (width 0.25) (layer "B.Cu") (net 11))
 (segment (start 149.86 104.14) (end 149.86 91.44) (width 0.25) (layer "B.Cu") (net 11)))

